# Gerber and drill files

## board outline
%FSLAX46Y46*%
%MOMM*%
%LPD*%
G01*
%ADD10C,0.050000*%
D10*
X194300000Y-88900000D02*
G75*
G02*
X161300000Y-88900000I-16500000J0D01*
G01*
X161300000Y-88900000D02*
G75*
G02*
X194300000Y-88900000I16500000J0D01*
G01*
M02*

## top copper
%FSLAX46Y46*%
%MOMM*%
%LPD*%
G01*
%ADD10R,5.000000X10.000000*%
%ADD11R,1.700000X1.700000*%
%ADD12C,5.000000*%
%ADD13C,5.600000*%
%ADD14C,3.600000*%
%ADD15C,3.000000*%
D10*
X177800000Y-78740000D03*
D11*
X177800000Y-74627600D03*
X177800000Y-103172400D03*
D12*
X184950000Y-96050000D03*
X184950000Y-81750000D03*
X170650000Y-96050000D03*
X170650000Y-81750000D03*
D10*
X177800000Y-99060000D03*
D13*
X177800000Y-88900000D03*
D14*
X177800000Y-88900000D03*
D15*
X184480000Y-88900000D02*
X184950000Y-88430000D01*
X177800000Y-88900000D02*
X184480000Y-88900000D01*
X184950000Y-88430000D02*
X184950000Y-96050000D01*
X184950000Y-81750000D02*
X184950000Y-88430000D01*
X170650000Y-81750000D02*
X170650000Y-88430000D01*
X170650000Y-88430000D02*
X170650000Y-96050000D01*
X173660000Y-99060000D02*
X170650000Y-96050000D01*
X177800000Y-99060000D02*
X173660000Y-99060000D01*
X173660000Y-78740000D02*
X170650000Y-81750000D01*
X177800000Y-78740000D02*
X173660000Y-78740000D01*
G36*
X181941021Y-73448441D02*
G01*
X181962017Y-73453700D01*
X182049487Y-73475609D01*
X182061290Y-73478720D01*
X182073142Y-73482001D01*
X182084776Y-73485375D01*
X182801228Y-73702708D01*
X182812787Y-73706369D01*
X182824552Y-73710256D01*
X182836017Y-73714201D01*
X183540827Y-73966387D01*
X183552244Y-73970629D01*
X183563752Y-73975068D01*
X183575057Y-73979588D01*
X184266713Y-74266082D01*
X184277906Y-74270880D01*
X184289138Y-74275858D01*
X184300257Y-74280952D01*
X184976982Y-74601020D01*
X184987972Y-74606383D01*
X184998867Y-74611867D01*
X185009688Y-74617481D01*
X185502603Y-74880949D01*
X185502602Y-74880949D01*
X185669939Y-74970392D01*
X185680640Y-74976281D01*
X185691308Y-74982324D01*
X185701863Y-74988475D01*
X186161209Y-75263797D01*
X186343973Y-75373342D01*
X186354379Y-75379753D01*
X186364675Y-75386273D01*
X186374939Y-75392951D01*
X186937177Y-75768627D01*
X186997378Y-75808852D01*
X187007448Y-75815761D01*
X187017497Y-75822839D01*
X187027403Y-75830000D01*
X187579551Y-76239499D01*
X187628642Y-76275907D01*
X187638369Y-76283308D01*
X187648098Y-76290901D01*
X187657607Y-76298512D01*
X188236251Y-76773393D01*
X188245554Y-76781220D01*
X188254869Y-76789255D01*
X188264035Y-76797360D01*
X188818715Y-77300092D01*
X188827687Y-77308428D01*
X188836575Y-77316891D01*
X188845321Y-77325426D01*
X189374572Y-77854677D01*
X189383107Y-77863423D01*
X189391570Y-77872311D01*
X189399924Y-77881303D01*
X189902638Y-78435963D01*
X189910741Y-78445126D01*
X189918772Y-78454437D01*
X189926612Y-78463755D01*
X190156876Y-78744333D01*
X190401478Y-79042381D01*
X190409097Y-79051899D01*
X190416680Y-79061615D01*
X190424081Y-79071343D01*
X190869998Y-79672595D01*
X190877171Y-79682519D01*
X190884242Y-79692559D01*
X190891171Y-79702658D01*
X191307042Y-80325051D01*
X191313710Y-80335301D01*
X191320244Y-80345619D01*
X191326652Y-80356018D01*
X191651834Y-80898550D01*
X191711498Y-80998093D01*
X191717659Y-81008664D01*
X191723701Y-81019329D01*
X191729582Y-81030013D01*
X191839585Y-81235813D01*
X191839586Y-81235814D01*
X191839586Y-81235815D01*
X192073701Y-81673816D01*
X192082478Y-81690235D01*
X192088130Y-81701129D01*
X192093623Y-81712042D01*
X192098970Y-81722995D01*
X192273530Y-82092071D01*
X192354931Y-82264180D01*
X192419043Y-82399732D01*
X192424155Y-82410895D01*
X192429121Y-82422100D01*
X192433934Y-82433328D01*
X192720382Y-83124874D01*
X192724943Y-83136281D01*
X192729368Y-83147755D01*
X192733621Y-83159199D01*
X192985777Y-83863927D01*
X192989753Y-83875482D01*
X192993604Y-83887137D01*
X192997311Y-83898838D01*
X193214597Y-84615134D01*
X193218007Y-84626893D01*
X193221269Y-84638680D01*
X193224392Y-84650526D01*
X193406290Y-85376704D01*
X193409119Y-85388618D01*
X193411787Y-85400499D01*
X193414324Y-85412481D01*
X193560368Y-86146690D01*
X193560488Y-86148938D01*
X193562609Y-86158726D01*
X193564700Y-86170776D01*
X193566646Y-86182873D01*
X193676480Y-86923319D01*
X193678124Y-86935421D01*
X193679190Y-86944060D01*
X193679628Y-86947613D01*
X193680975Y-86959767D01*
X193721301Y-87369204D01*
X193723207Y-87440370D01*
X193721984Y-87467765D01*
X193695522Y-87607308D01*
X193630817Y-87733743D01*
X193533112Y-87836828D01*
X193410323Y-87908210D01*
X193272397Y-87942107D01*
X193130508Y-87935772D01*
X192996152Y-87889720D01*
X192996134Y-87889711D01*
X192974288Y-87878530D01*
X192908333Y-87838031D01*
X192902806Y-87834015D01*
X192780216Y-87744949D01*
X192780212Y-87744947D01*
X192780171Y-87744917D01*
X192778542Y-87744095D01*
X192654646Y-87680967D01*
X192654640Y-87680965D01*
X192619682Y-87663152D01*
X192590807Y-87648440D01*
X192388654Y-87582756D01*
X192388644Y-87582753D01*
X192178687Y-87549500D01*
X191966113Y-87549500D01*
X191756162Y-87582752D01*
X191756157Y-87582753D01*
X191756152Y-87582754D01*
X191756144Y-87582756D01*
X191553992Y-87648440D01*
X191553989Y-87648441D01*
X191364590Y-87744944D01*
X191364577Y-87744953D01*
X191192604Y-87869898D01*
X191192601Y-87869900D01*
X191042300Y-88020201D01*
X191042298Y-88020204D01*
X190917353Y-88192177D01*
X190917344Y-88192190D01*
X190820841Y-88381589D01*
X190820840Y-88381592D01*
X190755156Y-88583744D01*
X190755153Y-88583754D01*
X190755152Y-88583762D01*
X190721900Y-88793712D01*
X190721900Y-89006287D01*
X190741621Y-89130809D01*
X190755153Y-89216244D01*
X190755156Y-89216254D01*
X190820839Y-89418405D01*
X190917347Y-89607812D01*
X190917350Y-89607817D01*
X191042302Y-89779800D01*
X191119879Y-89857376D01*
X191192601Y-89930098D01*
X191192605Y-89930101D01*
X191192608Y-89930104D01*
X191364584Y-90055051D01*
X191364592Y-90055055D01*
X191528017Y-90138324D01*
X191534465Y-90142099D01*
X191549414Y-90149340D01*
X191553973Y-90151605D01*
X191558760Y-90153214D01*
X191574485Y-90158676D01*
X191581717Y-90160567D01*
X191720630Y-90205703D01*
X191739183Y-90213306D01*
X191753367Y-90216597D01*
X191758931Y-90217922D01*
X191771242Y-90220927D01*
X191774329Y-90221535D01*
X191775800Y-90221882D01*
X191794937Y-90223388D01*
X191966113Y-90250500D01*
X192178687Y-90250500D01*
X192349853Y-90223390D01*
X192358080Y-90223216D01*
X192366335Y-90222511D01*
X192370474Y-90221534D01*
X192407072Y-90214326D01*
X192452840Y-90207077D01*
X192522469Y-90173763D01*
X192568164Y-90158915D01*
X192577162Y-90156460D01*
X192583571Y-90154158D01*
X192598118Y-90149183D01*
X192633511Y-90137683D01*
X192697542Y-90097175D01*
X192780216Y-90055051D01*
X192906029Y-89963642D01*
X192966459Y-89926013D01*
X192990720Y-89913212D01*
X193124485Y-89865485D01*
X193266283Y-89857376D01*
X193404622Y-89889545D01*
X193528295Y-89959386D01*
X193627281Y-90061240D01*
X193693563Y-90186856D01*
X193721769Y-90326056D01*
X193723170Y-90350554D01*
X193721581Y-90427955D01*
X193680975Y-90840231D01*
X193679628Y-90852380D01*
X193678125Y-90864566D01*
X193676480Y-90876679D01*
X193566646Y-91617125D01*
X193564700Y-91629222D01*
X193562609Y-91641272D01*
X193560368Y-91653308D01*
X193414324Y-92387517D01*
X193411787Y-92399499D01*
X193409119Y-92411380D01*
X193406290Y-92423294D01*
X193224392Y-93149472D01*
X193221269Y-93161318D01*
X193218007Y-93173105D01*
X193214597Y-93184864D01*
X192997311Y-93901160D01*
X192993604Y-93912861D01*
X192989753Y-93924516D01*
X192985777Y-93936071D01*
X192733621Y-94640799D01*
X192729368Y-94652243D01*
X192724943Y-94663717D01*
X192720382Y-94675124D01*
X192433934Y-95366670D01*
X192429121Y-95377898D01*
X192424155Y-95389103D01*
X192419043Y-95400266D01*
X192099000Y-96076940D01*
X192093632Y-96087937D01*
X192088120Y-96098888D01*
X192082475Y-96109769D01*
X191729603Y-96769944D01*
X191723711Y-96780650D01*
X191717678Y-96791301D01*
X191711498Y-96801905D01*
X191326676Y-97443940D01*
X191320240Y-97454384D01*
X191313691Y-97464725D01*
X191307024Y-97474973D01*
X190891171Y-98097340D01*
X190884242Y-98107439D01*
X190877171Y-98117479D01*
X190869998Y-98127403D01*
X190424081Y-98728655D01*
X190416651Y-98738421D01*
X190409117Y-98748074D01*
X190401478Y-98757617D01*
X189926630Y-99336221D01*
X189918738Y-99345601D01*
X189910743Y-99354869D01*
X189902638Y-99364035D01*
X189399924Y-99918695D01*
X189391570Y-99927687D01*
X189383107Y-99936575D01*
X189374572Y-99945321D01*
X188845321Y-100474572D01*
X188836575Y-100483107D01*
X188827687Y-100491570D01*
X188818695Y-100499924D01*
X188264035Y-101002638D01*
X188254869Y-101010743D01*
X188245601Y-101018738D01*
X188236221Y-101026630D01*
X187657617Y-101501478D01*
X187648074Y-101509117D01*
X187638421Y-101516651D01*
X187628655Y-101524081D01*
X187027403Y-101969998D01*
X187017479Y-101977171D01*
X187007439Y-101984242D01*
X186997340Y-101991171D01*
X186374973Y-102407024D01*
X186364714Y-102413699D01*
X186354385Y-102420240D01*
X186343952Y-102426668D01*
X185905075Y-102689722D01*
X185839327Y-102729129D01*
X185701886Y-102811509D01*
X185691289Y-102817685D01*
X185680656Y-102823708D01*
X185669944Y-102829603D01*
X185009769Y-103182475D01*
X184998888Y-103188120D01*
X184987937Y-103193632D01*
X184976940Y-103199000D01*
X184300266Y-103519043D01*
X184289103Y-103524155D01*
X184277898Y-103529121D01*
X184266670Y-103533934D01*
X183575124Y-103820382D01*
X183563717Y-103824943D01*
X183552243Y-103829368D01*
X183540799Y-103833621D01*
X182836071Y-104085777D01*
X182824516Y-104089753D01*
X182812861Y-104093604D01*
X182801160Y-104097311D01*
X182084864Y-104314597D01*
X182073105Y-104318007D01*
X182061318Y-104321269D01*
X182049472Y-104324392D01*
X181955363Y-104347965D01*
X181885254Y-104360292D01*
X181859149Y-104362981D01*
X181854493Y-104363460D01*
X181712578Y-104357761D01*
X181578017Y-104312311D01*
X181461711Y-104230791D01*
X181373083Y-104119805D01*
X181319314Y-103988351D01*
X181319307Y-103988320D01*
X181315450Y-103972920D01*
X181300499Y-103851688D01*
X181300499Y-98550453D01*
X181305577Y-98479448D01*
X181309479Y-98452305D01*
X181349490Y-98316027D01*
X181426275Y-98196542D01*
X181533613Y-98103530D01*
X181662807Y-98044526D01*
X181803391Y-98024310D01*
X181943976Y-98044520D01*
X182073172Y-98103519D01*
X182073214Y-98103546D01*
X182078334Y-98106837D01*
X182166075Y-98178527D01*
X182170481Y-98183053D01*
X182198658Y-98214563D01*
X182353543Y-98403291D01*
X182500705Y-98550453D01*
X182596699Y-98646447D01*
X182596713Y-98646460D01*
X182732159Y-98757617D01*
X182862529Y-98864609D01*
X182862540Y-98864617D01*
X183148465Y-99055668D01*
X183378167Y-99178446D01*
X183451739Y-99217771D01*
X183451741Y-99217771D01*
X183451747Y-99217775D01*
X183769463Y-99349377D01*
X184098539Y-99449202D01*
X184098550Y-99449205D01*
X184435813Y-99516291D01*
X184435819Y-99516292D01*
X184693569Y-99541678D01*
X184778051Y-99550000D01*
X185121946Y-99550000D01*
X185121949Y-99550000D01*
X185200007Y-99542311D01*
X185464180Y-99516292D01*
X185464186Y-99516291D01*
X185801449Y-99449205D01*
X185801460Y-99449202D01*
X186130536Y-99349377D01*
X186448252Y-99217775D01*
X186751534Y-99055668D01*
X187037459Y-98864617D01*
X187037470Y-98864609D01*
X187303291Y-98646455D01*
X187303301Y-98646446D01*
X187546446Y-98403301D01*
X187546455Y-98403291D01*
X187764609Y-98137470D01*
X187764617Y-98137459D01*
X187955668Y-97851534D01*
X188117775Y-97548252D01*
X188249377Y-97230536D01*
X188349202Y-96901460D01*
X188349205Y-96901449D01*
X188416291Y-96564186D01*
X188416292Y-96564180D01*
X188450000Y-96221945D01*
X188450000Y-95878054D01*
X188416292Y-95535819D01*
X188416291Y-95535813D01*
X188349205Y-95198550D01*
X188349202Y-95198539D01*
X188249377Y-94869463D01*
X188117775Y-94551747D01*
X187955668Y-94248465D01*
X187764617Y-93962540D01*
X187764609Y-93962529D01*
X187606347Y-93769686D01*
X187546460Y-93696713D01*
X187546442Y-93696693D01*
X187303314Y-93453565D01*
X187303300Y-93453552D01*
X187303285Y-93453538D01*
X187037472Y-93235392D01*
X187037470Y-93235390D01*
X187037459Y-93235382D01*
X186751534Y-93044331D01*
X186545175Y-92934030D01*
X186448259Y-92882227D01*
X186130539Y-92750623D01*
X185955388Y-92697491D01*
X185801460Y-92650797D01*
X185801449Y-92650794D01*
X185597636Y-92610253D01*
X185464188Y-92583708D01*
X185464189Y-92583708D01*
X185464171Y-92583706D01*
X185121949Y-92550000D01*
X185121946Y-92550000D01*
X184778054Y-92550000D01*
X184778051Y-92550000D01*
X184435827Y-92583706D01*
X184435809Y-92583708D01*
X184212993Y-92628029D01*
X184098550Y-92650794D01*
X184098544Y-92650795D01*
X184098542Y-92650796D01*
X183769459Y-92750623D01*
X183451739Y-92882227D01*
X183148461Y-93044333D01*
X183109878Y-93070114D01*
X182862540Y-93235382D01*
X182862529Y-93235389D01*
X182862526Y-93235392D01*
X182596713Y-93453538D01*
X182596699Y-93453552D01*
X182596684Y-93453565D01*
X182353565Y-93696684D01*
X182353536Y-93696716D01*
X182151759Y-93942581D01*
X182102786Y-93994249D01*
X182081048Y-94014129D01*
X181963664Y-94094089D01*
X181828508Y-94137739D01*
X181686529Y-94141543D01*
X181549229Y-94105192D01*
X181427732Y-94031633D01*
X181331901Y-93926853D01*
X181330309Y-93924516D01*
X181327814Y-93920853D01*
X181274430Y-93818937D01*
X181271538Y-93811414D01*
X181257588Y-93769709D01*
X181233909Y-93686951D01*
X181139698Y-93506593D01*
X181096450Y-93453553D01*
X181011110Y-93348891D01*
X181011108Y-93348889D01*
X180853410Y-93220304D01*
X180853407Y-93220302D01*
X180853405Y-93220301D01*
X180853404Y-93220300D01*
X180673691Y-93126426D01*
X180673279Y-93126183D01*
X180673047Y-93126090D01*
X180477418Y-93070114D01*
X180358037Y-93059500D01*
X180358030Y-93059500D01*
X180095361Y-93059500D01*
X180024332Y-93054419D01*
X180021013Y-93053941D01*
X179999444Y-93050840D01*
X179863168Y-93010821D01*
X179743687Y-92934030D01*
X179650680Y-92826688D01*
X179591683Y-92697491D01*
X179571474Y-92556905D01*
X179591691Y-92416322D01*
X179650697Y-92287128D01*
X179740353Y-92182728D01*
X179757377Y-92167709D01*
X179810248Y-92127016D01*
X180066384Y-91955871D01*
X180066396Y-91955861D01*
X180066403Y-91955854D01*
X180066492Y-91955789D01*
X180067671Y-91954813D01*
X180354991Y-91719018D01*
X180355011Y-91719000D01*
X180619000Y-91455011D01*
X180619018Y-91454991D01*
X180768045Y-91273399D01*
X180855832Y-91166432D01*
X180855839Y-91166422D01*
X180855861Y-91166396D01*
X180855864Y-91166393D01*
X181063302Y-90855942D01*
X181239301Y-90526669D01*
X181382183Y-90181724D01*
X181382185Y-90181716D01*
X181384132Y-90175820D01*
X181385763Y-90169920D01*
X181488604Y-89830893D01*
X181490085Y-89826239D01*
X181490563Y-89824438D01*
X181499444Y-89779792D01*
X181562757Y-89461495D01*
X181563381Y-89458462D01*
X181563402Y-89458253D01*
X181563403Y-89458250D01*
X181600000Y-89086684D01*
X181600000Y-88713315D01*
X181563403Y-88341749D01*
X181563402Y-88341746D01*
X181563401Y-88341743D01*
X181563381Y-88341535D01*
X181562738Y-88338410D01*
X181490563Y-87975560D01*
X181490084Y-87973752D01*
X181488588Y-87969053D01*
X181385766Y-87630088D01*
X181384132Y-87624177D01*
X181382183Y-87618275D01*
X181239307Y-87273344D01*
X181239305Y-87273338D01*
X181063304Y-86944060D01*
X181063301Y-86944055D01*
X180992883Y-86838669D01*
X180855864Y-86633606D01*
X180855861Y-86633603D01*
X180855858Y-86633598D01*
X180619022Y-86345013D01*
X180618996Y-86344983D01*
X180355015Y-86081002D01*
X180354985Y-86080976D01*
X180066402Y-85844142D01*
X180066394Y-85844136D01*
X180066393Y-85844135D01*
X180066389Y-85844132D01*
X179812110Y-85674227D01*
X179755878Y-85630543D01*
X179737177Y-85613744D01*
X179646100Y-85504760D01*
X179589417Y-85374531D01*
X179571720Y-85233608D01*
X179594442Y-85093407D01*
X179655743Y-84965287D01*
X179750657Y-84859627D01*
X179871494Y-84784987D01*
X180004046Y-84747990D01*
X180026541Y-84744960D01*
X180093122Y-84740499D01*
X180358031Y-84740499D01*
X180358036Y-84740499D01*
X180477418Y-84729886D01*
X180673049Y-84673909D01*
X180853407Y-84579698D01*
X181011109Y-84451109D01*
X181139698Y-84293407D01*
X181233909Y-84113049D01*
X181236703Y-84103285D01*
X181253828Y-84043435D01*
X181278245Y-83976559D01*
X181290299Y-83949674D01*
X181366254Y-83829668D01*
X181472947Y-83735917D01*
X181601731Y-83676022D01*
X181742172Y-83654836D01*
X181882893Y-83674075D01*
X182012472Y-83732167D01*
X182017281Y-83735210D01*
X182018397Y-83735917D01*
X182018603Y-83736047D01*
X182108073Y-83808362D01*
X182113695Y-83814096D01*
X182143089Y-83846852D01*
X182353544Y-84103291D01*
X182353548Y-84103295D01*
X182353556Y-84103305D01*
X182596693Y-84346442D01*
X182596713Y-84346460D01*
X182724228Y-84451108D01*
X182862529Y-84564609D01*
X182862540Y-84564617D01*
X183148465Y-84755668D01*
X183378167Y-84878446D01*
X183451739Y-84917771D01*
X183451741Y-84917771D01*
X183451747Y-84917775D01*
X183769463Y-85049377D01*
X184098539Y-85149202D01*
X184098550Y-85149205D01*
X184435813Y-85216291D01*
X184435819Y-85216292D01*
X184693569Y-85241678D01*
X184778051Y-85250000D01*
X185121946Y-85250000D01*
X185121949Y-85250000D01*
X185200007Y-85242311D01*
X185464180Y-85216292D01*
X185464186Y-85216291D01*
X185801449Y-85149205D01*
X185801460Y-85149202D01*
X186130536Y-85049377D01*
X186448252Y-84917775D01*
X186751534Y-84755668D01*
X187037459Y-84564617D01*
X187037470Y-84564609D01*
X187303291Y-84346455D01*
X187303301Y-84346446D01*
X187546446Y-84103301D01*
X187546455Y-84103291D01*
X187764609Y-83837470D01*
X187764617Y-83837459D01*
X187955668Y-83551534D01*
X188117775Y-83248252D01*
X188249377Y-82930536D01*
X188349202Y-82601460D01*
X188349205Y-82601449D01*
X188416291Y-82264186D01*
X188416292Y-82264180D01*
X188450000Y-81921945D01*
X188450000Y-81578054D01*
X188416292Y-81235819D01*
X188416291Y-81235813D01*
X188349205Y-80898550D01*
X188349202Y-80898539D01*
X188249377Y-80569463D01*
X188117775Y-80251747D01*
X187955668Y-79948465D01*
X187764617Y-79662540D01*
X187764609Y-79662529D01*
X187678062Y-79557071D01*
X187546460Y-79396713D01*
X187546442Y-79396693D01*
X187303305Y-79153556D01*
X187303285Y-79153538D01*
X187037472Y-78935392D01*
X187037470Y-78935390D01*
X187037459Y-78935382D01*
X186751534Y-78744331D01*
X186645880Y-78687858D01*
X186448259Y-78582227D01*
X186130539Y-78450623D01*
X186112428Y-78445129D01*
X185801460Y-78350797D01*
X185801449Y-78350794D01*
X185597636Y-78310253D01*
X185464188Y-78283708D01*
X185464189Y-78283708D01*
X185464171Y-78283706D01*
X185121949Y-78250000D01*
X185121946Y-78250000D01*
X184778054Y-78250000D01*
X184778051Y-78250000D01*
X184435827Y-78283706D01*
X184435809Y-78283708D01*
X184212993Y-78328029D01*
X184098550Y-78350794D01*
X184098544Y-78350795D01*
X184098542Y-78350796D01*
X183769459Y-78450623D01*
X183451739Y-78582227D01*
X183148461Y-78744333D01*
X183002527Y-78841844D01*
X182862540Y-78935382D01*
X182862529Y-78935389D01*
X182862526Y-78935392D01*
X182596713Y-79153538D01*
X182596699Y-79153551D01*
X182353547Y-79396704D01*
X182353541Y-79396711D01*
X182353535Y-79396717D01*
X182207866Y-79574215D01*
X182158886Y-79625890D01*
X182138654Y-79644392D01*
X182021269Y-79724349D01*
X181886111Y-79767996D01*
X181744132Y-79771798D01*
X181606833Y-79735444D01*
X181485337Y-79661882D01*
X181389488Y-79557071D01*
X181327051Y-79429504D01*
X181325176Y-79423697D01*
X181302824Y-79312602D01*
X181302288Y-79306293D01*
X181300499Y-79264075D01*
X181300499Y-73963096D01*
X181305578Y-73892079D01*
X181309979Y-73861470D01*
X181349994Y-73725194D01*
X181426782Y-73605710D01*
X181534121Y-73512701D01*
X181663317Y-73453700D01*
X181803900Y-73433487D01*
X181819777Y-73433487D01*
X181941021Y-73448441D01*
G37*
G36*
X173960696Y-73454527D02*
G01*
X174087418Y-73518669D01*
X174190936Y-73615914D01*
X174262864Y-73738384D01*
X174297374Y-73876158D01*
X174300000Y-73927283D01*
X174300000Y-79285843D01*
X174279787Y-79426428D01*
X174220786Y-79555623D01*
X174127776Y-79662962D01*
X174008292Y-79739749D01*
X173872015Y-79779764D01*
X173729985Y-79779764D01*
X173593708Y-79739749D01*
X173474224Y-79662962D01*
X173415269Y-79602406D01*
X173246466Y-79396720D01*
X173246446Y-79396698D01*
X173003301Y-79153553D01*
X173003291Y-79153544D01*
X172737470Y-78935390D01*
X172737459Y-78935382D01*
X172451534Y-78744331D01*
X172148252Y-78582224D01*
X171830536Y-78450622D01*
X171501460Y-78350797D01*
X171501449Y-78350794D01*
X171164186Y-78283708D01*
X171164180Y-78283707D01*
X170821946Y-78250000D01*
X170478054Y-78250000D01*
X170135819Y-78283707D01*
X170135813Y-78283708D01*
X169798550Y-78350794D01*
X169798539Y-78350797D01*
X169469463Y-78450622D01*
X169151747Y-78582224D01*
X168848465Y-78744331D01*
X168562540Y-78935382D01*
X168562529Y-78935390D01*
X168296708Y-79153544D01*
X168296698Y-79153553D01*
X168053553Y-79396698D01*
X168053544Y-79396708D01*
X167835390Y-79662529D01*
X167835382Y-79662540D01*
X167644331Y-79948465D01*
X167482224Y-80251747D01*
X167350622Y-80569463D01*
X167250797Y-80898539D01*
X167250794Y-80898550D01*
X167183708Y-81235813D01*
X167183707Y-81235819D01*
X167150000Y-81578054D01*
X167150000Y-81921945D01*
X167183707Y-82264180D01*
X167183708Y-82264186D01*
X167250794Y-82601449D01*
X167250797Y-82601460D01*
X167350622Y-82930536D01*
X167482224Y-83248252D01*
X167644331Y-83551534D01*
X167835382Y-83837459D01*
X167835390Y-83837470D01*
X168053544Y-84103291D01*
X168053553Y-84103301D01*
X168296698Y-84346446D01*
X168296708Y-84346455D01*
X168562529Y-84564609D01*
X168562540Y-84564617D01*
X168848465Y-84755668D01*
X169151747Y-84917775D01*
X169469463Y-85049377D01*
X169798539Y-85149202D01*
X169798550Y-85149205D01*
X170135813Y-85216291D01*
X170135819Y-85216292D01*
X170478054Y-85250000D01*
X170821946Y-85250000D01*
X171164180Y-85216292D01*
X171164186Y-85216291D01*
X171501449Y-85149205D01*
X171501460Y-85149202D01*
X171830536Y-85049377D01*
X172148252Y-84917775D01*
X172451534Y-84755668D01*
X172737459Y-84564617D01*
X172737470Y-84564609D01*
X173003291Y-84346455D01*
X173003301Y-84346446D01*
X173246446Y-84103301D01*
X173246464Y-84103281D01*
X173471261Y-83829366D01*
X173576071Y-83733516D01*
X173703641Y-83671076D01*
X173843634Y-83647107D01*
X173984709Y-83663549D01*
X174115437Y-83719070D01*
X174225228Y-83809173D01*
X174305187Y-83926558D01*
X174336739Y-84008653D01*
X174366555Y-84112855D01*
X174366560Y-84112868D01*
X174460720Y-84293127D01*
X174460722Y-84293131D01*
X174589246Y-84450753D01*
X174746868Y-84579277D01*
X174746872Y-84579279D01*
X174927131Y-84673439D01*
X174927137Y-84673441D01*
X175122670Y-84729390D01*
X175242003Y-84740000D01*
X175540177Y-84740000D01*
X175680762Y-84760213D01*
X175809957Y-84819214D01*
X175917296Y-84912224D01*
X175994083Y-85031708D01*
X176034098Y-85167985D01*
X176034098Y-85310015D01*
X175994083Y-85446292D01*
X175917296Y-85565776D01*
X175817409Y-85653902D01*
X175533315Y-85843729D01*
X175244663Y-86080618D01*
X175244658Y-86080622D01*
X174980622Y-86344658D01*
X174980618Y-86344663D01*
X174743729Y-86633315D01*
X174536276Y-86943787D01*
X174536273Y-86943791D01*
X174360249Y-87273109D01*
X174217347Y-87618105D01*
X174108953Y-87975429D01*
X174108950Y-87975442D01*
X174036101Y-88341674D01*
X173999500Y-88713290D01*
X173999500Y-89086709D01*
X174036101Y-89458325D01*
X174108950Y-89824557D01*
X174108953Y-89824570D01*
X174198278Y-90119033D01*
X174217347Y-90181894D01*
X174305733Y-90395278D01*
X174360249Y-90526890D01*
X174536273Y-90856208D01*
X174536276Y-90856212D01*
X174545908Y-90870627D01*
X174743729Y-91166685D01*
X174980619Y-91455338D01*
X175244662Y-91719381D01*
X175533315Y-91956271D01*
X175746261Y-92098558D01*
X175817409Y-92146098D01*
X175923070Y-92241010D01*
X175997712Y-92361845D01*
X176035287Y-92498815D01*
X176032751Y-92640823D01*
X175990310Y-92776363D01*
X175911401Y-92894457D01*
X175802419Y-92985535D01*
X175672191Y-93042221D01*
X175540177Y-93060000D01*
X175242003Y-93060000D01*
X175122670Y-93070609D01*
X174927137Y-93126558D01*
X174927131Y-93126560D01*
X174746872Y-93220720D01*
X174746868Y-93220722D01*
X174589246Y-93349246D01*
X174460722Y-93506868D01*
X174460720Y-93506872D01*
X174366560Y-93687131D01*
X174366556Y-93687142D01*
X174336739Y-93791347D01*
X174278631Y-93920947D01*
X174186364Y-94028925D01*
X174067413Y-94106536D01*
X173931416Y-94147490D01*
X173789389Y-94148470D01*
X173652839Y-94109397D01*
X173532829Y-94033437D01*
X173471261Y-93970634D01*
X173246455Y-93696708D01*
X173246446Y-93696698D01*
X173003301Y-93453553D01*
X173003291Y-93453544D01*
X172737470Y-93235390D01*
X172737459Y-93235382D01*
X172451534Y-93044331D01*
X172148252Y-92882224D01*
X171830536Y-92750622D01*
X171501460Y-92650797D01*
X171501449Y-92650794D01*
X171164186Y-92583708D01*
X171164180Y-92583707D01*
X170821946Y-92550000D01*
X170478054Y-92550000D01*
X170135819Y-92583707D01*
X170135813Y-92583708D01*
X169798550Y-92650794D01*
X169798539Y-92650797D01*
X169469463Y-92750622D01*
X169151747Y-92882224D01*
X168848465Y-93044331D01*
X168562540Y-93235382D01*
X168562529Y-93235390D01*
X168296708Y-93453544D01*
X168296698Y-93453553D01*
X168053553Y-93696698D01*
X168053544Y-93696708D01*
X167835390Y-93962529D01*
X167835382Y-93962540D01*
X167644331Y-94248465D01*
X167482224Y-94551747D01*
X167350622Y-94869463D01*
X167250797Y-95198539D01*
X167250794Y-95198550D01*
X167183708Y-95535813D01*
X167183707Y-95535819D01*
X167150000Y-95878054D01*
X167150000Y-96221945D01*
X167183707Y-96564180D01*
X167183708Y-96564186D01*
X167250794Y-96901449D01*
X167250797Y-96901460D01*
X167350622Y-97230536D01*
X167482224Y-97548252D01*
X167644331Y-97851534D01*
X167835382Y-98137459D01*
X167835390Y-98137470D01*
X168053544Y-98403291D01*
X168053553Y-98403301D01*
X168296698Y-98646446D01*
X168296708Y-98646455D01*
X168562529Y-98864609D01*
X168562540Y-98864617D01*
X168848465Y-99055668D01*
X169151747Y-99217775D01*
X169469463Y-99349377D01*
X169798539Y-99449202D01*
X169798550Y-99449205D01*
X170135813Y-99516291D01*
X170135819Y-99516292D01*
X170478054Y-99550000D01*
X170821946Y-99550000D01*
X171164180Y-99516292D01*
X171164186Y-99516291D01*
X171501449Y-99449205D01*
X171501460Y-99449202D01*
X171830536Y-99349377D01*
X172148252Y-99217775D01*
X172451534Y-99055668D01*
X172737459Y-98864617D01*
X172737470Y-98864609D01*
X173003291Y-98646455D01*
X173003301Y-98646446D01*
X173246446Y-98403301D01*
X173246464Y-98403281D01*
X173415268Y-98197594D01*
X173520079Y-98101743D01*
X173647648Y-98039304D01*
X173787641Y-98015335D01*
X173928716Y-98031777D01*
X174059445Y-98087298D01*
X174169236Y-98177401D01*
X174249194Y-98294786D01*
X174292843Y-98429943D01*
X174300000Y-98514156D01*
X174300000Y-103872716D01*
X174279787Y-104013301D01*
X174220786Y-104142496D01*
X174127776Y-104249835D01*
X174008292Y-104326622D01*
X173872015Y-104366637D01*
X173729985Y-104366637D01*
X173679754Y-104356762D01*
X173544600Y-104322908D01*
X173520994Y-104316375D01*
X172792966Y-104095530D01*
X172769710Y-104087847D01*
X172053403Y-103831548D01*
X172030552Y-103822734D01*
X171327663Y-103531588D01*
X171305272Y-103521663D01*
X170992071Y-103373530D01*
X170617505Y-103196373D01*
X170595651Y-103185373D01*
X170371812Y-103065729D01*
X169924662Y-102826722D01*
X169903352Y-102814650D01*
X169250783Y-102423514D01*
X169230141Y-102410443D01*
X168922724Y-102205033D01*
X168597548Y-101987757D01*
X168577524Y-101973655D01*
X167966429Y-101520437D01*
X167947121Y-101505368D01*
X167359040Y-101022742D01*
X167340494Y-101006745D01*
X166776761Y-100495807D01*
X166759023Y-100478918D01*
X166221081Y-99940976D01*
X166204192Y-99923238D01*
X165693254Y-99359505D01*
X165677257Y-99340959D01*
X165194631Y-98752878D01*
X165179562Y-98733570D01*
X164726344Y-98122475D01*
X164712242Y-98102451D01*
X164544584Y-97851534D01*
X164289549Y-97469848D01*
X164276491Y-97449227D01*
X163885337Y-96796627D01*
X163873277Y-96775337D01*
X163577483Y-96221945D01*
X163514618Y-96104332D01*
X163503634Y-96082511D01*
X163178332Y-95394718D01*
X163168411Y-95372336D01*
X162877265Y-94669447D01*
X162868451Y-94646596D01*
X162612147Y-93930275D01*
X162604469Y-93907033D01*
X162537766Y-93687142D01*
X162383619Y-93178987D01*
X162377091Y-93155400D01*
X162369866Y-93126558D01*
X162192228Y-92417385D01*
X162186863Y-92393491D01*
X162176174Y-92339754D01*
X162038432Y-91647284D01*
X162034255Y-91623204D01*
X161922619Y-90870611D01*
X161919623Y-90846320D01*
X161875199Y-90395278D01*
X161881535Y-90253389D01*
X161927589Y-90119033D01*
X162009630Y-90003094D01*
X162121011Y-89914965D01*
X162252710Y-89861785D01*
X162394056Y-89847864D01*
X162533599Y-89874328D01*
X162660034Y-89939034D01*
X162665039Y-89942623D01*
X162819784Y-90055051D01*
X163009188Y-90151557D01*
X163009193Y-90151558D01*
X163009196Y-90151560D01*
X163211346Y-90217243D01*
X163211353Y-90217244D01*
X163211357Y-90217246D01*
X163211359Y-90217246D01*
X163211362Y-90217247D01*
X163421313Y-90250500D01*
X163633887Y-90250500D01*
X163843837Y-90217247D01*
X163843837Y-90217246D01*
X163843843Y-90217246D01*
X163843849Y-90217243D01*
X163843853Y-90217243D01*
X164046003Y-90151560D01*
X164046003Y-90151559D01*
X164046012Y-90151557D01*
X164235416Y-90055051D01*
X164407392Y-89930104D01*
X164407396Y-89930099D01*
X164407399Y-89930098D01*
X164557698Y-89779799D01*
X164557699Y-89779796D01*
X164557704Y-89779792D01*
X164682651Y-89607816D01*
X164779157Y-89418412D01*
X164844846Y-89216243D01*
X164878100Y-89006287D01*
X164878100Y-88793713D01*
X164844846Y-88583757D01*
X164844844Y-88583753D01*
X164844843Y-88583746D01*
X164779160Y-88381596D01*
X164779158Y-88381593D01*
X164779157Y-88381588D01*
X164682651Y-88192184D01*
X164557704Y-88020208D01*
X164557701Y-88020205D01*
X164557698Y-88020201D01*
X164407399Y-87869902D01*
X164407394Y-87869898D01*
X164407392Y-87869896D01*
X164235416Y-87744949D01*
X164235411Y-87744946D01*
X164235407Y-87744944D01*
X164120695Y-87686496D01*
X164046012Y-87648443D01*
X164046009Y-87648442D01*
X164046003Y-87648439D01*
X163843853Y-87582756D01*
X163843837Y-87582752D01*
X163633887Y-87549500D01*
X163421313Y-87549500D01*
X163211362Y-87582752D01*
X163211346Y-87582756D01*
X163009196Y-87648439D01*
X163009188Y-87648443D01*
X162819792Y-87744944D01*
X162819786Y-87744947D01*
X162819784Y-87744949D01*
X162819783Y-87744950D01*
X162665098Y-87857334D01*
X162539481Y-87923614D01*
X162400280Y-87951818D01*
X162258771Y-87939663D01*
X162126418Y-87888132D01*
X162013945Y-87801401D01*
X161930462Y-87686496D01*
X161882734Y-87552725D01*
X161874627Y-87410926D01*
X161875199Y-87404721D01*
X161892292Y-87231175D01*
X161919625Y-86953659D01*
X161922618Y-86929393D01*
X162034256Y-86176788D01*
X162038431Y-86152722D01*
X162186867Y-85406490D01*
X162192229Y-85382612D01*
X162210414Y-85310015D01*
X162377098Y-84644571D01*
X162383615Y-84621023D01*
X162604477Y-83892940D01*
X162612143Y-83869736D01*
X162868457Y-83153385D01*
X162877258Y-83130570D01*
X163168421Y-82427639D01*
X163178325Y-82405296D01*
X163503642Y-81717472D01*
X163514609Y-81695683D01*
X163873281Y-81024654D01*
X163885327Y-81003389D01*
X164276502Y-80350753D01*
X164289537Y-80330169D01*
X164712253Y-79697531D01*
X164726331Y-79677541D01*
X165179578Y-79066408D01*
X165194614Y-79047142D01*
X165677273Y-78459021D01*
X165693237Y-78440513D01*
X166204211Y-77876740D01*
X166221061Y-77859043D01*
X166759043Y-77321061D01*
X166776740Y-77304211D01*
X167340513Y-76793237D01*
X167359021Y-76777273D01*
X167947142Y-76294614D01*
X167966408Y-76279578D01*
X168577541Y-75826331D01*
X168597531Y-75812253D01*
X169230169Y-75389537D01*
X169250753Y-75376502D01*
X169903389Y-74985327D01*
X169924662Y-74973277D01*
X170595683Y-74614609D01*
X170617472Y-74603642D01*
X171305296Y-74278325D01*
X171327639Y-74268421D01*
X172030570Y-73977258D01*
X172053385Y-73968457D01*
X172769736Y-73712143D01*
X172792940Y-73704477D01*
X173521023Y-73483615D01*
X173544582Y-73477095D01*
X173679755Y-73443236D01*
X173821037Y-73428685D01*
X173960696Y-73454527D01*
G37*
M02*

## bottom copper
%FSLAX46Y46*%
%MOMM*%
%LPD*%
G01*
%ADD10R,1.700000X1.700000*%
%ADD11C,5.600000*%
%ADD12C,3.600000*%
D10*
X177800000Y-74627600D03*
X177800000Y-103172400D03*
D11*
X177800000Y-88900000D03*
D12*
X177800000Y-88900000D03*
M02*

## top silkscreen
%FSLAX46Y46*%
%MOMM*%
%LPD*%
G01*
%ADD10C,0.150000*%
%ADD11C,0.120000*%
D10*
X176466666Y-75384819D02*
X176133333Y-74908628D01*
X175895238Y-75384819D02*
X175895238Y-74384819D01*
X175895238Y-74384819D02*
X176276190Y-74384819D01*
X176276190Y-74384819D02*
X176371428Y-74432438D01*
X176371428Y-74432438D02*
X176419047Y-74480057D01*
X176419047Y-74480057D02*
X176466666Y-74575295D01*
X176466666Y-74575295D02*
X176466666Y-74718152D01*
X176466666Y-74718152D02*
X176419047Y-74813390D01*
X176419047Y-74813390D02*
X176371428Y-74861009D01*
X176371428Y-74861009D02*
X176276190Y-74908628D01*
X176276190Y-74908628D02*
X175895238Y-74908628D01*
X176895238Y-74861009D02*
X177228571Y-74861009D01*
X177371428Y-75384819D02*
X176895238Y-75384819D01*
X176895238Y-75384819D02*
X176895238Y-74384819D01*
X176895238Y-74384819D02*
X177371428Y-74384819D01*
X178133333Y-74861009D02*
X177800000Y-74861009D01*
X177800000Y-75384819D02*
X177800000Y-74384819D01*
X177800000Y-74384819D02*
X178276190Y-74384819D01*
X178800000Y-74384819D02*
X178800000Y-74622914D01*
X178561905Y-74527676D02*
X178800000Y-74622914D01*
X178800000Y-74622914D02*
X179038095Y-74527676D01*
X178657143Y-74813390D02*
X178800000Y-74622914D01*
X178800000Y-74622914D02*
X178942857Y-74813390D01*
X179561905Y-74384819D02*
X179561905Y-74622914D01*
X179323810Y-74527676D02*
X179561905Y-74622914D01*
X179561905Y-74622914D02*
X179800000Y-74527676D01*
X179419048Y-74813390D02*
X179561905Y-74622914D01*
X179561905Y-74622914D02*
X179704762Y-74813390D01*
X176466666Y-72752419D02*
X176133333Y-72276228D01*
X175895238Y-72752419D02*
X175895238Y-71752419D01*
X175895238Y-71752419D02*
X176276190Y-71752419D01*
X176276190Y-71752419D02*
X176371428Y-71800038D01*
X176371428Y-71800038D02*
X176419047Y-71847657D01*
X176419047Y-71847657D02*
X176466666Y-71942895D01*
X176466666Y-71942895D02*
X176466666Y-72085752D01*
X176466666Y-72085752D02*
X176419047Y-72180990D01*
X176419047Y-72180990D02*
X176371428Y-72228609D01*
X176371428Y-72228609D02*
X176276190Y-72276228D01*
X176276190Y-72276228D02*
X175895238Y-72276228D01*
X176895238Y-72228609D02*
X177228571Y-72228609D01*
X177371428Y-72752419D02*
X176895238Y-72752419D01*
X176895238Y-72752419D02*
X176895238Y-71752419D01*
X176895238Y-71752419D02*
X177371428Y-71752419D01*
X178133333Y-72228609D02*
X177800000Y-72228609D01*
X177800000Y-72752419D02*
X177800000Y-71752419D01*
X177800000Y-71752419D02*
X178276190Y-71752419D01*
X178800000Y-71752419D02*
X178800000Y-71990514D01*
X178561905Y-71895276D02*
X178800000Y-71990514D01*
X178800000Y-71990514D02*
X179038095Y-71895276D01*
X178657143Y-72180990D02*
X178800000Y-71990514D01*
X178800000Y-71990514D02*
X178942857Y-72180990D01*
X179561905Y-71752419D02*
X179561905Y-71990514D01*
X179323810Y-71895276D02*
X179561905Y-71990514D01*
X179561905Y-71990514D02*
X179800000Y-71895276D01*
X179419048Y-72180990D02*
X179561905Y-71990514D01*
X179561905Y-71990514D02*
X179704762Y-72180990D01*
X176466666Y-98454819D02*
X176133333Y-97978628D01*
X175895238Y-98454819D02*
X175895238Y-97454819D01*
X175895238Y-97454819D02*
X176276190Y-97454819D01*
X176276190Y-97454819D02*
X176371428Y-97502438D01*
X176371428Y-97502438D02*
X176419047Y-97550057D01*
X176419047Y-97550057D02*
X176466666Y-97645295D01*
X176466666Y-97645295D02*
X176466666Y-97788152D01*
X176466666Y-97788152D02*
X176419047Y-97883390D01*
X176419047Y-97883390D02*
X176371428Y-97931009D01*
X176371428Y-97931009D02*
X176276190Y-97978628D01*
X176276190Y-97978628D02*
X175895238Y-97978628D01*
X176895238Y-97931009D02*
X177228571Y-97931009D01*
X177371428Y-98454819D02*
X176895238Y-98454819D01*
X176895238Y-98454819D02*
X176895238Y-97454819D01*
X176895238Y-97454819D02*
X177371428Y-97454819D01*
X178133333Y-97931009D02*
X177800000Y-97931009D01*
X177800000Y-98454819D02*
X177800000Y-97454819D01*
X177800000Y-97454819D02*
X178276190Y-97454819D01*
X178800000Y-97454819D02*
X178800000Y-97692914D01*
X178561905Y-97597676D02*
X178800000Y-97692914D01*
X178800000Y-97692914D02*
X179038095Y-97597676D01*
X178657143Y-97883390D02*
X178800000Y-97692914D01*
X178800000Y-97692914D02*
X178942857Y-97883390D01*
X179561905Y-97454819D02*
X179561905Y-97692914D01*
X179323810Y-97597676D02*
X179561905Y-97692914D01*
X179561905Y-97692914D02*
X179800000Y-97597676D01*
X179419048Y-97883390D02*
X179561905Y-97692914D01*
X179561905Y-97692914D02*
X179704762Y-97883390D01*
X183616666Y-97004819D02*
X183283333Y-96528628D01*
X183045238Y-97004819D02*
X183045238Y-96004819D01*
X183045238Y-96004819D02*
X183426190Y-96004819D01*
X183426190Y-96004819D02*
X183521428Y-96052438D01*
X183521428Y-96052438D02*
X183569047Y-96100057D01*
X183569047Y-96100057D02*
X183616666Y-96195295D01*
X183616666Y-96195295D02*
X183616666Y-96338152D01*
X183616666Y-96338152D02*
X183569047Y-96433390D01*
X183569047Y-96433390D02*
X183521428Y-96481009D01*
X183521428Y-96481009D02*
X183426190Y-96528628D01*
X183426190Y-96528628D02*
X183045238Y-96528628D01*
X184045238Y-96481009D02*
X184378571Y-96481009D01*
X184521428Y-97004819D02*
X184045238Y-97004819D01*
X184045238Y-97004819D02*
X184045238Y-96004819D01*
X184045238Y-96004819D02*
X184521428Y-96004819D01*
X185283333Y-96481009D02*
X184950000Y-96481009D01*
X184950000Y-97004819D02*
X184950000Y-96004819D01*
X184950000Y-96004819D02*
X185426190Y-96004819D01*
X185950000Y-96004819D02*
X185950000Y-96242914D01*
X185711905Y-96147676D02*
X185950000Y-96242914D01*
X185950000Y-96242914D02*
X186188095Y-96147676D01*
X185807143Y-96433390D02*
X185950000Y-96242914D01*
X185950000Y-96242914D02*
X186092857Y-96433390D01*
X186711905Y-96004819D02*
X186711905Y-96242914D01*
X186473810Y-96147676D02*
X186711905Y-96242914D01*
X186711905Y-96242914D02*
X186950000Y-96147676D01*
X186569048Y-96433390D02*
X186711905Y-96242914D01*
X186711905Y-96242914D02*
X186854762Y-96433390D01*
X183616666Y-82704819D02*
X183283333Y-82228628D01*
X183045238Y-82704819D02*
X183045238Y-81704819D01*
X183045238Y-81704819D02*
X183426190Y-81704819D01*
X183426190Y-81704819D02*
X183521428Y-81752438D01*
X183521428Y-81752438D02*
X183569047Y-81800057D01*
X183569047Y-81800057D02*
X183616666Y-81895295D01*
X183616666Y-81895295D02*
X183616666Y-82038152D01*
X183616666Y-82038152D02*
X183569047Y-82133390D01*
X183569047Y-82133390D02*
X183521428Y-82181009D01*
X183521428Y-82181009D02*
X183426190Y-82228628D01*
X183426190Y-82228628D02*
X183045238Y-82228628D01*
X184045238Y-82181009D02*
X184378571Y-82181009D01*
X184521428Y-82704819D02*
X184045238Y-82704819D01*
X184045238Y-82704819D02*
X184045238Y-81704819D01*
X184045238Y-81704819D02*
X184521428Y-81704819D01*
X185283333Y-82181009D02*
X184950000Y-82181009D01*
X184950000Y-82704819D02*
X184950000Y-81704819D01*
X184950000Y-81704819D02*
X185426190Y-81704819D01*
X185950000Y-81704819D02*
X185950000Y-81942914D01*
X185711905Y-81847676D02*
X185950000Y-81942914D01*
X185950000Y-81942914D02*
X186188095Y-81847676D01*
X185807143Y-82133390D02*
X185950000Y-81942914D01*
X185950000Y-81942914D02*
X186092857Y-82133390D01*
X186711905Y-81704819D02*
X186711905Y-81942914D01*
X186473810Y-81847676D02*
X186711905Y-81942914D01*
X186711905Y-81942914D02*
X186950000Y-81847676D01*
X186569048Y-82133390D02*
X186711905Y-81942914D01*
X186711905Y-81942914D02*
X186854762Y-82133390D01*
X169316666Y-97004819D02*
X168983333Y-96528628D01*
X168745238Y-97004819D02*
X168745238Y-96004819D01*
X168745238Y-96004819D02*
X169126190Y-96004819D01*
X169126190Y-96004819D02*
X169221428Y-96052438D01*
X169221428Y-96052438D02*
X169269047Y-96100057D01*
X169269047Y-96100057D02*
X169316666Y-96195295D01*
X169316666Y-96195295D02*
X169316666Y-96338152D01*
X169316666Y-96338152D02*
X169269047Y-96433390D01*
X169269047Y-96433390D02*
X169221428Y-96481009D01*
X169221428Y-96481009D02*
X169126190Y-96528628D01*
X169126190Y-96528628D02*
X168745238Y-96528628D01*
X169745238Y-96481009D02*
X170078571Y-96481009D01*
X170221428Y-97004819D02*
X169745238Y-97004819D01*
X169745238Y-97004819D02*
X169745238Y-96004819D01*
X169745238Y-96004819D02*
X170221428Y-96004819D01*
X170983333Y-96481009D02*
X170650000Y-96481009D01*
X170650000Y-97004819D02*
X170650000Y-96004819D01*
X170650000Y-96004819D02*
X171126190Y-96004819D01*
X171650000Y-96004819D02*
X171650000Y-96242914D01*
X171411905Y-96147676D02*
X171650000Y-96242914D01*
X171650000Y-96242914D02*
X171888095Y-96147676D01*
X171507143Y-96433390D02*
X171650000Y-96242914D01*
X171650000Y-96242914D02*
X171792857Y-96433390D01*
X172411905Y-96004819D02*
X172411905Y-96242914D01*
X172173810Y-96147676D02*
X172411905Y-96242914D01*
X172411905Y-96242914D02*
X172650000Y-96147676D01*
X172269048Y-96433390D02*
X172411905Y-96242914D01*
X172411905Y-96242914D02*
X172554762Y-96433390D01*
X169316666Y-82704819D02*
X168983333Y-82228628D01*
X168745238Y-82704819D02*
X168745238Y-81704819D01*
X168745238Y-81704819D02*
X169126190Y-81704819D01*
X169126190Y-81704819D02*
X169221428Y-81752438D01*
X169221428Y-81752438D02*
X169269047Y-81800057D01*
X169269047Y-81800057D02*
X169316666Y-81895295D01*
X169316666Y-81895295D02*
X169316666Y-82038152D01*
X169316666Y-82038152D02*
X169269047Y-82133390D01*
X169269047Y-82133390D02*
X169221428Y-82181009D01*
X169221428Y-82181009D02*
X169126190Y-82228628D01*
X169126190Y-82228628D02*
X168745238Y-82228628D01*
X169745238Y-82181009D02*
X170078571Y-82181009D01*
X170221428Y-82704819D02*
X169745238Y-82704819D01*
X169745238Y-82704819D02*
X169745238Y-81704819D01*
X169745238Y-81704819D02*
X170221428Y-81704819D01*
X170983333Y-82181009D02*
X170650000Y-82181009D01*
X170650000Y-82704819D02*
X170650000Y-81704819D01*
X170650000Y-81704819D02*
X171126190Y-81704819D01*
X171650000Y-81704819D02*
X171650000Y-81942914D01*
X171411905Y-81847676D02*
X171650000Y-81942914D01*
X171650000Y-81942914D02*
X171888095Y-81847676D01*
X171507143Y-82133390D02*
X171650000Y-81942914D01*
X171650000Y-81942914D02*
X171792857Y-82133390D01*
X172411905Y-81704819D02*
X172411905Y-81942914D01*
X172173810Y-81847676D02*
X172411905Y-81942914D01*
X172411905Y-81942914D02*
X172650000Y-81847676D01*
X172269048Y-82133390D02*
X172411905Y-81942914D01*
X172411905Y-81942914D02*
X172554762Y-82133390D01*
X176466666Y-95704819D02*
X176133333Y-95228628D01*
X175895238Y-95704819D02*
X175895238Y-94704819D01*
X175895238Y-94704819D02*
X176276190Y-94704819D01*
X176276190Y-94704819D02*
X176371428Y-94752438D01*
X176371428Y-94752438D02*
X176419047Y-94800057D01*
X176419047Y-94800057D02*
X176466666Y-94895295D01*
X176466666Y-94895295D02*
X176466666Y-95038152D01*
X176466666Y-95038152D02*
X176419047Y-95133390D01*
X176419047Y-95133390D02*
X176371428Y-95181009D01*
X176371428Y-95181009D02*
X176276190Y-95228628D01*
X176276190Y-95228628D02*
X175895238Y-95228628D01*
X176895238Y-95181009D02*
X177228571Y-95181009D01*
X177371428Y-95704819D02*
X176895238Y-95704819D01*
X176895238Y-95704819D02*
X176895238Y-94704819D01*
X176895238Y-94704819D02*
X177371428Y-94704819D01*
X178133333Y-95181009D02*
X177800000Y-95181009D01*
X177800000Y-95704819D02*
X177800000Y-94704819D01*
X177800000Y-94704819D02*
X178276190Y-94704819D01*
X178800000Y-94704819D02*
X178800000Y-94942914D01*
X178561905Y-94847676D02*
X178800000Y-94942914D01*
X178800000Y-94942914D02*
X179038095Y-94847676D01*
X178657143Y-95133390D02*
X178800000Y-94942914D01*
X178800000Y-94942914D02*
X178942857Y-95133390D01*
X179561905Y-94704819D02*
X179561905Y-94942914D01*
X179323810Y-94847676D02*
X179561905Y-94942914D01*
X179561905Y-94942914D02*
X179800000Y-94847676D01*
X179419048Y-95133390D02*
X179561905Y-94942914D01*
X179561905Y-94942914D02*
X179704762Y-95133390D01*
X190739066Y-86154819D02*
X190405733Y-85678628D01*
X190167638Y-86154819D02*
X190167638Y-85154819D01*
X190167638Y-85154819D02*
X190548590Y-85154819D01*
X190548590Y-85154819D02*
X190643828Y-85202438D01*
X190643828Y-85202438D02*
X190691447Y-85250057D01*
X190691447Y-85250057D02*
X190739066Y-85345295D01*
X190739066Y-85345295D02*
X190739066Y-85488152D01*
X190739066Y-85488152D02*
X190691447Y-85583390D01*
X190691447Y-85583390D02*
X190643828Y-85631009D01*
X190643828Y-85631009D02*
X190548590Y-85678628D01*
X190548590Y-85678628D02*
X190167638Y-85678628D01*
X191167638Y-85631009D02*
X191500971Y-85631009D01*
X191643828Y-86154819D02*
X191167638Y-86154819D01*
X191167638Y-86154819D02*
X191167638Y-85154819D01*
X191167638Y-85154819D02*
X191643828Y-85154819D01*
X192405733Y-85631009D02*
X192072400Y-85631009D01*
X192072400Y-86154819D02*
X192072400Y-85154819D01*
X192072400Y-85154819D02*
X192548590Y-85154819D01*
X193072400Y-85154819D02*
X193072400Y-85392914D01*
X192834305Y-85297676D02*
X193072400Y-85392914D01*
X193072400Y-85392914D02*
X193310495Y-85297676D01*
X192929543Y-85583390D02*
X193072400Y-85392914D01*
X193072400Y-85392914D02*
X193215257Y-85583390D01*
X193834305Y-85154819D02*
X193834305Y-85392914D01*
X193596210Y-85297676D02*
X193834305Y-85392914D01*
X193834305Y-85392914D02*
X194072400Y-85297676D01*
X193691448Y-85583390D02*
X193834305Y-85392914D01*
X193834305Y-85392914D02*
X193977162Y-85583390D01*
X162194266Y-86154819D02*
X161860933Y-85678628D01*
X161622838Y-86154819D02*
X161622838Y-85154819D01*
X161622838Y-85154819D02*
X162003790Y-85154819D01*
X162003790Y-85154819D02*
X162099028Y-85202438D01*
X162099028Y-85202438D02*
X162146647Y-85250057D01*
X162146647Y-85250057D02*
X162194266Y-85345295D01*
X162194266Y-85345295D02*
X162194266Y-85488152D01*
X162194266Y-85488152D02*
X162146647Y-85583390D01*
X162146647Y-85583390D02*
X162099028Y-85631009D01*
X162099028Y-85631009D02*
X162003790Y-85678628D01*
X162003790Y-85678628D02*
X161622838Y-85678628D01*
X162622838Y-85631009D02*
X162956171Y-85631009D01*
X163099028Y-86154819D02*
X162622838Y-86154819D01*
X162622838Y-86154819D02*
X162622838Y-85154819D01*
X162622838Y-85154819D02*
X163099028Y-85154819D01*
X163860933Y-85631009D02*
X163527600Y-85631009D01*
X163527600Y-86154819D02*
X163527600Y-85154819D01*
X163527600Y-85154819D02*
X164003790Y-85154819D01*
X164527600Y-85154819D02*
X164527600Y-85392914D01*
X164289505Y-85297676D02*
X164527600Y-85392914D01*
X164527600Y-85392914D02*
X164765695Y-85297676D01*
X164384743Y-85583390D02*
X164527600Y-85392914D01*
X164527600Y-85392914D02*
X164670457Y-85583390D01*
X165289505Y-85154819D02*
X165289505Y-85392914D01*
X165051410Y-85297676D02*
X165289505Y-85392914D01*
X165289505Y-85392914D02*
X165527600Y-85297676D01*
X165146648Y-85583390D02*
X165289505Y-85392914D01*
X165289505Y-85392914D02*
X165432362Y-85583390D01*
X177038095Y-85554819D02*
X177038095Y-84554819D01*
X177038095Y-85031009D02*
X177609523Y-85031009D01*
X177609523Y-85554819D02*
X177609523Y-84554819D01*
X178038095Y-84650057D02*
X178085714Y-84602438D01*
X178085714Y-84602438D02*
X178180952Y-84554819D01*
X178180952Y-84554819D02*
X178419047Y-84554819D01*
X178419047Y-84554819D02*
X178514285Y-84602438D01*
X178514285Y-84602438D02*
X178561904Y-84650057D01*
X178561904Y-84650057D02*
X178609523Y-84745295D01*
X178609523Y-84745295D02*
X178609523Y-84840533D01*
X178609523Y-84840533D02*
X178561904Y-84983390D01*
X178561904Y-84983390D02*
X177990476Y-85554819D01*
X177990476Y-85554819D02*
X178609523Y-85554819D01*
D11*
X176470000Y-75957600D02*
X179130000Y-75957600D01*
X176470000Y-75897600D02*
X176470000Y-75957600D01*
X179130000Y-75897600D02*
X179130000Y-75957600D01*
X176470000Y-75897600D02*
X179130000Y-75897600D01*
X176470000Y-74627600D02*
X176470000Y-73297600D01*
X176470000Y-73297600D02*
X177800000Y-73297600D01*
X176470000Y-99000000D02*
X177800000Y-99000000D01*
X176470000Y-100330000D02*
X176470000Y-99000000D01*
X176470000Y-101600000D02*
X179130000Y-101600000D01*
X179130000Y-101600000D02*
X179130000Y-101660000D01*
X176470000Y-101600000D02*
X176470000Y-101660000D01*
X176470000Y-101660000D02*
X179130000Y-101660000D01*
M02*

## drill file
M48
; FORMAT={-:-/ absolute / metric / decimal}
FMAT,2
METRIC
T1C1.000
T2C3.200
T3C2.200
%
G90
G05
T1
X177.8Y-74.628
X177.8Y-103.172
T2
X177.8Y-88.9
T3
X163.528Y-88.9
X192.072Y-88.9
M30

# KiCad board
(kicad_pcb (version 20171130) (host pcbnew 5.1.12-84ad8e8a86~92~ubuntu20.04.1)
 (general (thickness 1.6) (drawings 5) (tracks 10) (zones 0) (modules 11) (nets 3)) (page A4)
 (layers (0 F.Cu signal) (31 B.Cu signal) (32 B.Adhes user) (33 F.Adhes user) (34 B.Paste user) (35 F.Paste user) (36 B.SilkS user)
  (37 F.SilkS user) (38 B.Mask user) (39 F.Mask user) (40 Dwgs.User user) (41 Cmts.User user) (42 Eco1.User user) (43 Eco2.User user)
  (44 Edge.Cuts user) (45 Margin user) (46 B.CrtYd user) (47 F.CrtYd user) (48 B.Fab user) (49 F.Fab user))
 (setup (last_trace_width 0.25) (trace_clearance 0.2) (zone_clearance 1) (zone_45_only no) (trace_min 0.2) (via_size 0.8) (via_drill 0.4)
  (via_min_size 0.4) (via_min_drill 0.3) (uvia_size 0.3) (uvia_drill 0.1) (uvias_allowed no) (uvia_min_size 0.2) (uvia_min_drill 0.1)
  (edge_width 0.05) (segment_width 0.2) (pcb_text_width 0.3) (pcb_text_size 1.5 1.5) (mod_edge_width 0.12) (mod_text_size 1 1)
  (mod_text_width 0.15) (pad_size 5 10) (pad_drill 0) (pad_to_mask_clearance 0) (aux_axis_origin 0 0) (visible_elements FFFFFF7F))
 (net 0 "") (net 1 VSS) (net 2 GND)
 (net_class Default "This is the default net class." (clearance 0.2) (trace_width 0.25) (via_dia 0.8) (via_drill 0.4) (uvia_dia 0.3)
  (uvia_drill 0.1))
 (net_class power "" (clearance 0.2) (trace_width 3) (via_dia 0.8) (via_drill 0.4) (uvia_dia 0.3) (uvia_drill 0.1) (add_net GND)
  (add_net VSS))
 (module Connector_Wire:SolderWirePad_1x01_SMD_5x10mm (layer F.Cu) (at 177.8 78.74)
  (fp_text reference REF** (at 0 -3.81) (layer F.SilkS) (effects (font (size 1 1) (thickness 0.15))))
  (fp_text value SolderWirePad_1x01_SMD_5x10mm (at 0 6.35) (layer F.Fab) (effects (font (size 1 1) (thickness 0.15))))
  (pad 1 smd rect (at 0 0) (size 5 10) (layers F.Cu F.Paste F.Mask) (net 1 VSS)))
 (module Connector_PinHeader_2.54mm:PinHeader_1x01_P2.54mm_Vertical (layer F.Cu) (at 177.8 74.6276)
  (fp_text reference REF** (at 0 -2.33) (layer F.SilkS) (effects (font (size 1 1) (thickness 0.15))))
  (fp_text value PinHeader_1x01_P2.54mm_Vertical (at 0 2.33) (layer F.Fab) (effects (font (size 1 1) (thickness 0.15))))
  (fp_line (start -1.33 1.33) (end 1.33 1.33) (layer F.SilkS) (width 0.12))
  (fp_line (start -1.33 1.27) (end -1.33 1.33) (layer F.SilkS) (width 0.12))
  (fp_line (start 1.33 1.27) (end 1.33 1.33) (layer F.SilkS) (width 0.12))
  (fp_line (start -1.33 1.27) (end 1.33 1.27) (layer F.SilkS) (width 0.12))
  (fp_line (start -1.33 0) (end -1.33 -1.33) (layer F.SilkS) (width 0.12))
  (fp_line (start -1.33 -1.33) (end 0 -1.33) (layer F.SilkS) (width 0.12))
  (pad 1 thru_hole rect (at 0 0) (size 1.7 1.7) (drill 1) (layers *.Cu *.Mask) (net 1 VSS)))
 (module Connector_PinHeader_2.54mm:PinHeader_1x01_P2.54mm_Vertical (layer F.Cu) (at 177.8 100.33)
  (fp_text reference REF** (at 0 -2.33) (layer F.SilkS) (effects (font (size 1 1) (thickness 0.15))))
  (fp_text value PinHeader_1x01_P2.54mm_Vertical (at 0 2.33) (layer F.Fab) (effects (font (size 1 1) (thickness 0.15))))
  (fp_line (start -1.33 -1.33) (end 0 -1.33) (layer F.SilkS) (width 0.12))
  (fp_line (start -1.33 0) (end -1.33 -1.33) (layer F.SilkS) (width 0.12))
  (fp_line (start -1.33 1.27) (end 1.33 1.27) (layer F.SilkS) (width 0.12))
  (fp_line (start 1.33 1.27) (end 1.33 1.33) (layer F.SilkS) (width 0.12))
  (fp_line (start -1.33 1.27) (end -1.33 1.33) (layer F.SilkS) (width 0.12))
  (fp_line (start -1.33 1.33) (end 1.33 1.33) (layer F.SilkS) (width 0.12))
  (pad 1 thru_hole rect (at 0 2.8424) (size 1.7 1.7) (drill 1) (layers *.Cu *.Mask) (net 1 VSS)))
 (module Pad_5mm (layer F.Cu) (at 184.95 96.05)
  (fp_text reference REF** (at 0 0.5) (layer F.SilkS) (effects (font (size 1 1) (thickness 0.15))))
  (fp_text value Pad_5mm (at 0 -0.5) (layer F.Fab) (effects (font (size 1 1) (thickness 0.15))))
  (pad 1 smd circle (at 0 0) (size 5 5) (layers F.Cu F.Paste F.Mask) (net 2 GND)))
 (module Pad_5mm (layer F.Cu) (at 184.95 81.75)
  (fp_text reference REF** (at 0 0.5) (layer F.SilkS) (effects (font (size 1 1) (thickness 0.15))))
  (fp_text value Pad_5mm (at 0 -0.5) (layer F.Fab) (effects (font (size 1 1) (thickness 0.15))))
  (pad 1 smd circle (at 0 0) (size 5 5) (layers F.Cu F.Paste F.Mask) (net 2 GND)))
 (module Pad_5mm (layer F.Cu) (at 170.65 96.05)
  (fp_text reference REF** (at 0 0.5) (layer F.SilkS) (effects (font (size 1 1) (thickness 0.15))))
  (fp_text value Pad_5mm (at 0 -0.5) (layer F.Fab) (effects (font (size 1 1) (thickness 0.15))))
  (pad 1 smd circle (at 0 0) (size 5 5) (layers F.Cu F.Paste F.Mask) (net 1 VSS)))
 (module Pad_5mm (layer F.Cu) (at 170.65 81.75)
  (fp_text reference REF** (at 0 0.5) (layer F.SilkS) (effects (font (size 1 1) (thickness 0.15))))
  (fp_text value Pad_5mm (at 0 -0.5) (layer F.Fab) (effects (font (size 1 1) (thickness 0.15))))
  (pad 1 smd circle (at 0 0) (size 5 5) (layers F.Cu F.Paste F.Mask) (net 1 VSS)))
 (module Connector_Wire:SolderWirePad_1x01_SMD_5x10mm (layer F.Cu) (at 177.8 99.06)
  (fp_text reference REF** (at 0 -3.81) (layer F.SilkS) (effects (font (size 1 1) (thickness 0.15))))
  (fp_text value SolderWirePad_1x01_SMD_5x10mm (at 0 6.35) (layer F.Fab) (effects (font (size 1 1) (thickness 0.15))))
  (pad 1 smd rect (at 0 0) (size 5 10) (layers F.Cu F.Paste F.Mask) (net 1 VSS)))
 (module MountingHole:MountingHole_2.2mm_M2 (layer F.Cu) (at 192.0724 88.9)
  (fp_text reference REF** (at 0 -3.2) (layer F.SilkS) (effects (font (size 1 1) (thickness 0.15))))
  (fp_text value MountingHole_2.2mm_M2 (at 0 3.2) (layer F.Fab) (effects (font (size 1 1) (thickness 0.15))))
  (pad 1 np_thru_hole circle (at 0 0) (size 2.2 2.2) (drill 2.2) (layers *.Cu *.Mask)))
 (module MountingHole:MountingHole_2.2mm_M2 (layer F.Cu) (at 163.5276 88.9)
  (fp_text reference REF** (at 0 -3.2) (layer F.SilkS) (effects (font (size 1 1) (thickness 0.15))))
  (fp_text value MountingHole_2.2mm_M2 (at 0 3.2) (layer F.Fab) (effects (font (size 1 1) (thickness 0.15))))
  (pad 1 np_thru_hole circle (at 0 0) (size 2.2 2.2) (drill 2.2) (layers *.Cu *.Mask)))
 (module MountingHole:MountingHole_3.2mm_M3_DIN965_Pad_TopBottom (layer F.Cu) (at 177.8 88.9)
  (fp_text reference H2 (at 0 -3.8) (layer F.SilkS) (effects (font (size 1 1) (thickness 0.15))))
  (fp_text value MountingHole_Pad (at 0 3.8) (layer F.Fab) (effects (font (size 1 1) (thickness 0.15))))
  (pad 1 connect circle (at 0 0) (size 5.6 5.6) (layers B.Cu B.Mask) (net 2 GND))
  (pad 1 connect circle (at 0 0) (size 5.6 5.6) (layers F.Cu F.Mask) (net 2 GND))
  (pad 1 thru_hole circle (at 0 0) (size 3.6 3.6) (drill 3.2) (layers *.Cu *.Mask) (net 2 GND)))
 (gr_circle (center 177.8 88.9) (end 194.3 88.9) (layer Edge.Cuts) (width 0.05))
 (segment (start 184.48 88.9) (end 184.95 88.43) (width 3) (layer F.Cu) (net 2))
 (segment (start 177.8 88.9) (end 184.48 88.9) (width 3) (layer F.Cu) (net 2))
 (segment (start 184.95 88.43) (end 184.95 96.05) (width 3) (layer F.Cu) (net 2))
 (segment (start 184.95 81.75) (end 184.95 88.43) (width 3) (layer F.Cu) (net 2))
 (segment (start 170.65 81.75) (end 170.65 88.43) (width 3) (layer F.Cu) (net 1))
 (segment (start 170.65 88.43) (end 170.65 96.05) (width 3) (layer F.Cu) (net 1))
 (segment (start 173.66 99.06) (end 170.65 96.05) (width 3) (layer F.Cu) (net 1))
 (segment (start 177.8 99.06) (end 173.66 99.06) (width 3) (layer F.Cu) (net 1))
 (segment (start 173.66 78.74) (end 170.65 81.75) (width 3) (layer F.Cu) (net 1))
 (segment (start 177.8 78.74) (end 173.66 78.74) (width 3) (layer F.Cu) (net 1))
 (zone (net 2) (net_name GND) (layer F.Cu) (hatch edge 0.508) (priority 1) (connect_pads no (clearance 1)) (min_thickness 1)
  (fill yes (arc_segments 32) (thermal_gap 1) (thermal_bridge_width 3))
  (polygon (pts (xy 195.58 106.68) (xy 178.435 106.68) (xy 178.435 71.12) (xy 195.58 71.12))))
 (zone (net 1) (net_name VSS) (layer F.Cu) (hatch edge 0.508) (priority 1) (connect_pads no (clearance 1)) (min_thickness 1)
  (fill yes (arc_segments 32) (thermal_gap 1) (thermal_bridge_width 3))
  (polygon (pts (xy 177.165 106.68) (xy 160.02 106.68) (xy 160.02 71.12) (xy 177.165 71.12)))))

